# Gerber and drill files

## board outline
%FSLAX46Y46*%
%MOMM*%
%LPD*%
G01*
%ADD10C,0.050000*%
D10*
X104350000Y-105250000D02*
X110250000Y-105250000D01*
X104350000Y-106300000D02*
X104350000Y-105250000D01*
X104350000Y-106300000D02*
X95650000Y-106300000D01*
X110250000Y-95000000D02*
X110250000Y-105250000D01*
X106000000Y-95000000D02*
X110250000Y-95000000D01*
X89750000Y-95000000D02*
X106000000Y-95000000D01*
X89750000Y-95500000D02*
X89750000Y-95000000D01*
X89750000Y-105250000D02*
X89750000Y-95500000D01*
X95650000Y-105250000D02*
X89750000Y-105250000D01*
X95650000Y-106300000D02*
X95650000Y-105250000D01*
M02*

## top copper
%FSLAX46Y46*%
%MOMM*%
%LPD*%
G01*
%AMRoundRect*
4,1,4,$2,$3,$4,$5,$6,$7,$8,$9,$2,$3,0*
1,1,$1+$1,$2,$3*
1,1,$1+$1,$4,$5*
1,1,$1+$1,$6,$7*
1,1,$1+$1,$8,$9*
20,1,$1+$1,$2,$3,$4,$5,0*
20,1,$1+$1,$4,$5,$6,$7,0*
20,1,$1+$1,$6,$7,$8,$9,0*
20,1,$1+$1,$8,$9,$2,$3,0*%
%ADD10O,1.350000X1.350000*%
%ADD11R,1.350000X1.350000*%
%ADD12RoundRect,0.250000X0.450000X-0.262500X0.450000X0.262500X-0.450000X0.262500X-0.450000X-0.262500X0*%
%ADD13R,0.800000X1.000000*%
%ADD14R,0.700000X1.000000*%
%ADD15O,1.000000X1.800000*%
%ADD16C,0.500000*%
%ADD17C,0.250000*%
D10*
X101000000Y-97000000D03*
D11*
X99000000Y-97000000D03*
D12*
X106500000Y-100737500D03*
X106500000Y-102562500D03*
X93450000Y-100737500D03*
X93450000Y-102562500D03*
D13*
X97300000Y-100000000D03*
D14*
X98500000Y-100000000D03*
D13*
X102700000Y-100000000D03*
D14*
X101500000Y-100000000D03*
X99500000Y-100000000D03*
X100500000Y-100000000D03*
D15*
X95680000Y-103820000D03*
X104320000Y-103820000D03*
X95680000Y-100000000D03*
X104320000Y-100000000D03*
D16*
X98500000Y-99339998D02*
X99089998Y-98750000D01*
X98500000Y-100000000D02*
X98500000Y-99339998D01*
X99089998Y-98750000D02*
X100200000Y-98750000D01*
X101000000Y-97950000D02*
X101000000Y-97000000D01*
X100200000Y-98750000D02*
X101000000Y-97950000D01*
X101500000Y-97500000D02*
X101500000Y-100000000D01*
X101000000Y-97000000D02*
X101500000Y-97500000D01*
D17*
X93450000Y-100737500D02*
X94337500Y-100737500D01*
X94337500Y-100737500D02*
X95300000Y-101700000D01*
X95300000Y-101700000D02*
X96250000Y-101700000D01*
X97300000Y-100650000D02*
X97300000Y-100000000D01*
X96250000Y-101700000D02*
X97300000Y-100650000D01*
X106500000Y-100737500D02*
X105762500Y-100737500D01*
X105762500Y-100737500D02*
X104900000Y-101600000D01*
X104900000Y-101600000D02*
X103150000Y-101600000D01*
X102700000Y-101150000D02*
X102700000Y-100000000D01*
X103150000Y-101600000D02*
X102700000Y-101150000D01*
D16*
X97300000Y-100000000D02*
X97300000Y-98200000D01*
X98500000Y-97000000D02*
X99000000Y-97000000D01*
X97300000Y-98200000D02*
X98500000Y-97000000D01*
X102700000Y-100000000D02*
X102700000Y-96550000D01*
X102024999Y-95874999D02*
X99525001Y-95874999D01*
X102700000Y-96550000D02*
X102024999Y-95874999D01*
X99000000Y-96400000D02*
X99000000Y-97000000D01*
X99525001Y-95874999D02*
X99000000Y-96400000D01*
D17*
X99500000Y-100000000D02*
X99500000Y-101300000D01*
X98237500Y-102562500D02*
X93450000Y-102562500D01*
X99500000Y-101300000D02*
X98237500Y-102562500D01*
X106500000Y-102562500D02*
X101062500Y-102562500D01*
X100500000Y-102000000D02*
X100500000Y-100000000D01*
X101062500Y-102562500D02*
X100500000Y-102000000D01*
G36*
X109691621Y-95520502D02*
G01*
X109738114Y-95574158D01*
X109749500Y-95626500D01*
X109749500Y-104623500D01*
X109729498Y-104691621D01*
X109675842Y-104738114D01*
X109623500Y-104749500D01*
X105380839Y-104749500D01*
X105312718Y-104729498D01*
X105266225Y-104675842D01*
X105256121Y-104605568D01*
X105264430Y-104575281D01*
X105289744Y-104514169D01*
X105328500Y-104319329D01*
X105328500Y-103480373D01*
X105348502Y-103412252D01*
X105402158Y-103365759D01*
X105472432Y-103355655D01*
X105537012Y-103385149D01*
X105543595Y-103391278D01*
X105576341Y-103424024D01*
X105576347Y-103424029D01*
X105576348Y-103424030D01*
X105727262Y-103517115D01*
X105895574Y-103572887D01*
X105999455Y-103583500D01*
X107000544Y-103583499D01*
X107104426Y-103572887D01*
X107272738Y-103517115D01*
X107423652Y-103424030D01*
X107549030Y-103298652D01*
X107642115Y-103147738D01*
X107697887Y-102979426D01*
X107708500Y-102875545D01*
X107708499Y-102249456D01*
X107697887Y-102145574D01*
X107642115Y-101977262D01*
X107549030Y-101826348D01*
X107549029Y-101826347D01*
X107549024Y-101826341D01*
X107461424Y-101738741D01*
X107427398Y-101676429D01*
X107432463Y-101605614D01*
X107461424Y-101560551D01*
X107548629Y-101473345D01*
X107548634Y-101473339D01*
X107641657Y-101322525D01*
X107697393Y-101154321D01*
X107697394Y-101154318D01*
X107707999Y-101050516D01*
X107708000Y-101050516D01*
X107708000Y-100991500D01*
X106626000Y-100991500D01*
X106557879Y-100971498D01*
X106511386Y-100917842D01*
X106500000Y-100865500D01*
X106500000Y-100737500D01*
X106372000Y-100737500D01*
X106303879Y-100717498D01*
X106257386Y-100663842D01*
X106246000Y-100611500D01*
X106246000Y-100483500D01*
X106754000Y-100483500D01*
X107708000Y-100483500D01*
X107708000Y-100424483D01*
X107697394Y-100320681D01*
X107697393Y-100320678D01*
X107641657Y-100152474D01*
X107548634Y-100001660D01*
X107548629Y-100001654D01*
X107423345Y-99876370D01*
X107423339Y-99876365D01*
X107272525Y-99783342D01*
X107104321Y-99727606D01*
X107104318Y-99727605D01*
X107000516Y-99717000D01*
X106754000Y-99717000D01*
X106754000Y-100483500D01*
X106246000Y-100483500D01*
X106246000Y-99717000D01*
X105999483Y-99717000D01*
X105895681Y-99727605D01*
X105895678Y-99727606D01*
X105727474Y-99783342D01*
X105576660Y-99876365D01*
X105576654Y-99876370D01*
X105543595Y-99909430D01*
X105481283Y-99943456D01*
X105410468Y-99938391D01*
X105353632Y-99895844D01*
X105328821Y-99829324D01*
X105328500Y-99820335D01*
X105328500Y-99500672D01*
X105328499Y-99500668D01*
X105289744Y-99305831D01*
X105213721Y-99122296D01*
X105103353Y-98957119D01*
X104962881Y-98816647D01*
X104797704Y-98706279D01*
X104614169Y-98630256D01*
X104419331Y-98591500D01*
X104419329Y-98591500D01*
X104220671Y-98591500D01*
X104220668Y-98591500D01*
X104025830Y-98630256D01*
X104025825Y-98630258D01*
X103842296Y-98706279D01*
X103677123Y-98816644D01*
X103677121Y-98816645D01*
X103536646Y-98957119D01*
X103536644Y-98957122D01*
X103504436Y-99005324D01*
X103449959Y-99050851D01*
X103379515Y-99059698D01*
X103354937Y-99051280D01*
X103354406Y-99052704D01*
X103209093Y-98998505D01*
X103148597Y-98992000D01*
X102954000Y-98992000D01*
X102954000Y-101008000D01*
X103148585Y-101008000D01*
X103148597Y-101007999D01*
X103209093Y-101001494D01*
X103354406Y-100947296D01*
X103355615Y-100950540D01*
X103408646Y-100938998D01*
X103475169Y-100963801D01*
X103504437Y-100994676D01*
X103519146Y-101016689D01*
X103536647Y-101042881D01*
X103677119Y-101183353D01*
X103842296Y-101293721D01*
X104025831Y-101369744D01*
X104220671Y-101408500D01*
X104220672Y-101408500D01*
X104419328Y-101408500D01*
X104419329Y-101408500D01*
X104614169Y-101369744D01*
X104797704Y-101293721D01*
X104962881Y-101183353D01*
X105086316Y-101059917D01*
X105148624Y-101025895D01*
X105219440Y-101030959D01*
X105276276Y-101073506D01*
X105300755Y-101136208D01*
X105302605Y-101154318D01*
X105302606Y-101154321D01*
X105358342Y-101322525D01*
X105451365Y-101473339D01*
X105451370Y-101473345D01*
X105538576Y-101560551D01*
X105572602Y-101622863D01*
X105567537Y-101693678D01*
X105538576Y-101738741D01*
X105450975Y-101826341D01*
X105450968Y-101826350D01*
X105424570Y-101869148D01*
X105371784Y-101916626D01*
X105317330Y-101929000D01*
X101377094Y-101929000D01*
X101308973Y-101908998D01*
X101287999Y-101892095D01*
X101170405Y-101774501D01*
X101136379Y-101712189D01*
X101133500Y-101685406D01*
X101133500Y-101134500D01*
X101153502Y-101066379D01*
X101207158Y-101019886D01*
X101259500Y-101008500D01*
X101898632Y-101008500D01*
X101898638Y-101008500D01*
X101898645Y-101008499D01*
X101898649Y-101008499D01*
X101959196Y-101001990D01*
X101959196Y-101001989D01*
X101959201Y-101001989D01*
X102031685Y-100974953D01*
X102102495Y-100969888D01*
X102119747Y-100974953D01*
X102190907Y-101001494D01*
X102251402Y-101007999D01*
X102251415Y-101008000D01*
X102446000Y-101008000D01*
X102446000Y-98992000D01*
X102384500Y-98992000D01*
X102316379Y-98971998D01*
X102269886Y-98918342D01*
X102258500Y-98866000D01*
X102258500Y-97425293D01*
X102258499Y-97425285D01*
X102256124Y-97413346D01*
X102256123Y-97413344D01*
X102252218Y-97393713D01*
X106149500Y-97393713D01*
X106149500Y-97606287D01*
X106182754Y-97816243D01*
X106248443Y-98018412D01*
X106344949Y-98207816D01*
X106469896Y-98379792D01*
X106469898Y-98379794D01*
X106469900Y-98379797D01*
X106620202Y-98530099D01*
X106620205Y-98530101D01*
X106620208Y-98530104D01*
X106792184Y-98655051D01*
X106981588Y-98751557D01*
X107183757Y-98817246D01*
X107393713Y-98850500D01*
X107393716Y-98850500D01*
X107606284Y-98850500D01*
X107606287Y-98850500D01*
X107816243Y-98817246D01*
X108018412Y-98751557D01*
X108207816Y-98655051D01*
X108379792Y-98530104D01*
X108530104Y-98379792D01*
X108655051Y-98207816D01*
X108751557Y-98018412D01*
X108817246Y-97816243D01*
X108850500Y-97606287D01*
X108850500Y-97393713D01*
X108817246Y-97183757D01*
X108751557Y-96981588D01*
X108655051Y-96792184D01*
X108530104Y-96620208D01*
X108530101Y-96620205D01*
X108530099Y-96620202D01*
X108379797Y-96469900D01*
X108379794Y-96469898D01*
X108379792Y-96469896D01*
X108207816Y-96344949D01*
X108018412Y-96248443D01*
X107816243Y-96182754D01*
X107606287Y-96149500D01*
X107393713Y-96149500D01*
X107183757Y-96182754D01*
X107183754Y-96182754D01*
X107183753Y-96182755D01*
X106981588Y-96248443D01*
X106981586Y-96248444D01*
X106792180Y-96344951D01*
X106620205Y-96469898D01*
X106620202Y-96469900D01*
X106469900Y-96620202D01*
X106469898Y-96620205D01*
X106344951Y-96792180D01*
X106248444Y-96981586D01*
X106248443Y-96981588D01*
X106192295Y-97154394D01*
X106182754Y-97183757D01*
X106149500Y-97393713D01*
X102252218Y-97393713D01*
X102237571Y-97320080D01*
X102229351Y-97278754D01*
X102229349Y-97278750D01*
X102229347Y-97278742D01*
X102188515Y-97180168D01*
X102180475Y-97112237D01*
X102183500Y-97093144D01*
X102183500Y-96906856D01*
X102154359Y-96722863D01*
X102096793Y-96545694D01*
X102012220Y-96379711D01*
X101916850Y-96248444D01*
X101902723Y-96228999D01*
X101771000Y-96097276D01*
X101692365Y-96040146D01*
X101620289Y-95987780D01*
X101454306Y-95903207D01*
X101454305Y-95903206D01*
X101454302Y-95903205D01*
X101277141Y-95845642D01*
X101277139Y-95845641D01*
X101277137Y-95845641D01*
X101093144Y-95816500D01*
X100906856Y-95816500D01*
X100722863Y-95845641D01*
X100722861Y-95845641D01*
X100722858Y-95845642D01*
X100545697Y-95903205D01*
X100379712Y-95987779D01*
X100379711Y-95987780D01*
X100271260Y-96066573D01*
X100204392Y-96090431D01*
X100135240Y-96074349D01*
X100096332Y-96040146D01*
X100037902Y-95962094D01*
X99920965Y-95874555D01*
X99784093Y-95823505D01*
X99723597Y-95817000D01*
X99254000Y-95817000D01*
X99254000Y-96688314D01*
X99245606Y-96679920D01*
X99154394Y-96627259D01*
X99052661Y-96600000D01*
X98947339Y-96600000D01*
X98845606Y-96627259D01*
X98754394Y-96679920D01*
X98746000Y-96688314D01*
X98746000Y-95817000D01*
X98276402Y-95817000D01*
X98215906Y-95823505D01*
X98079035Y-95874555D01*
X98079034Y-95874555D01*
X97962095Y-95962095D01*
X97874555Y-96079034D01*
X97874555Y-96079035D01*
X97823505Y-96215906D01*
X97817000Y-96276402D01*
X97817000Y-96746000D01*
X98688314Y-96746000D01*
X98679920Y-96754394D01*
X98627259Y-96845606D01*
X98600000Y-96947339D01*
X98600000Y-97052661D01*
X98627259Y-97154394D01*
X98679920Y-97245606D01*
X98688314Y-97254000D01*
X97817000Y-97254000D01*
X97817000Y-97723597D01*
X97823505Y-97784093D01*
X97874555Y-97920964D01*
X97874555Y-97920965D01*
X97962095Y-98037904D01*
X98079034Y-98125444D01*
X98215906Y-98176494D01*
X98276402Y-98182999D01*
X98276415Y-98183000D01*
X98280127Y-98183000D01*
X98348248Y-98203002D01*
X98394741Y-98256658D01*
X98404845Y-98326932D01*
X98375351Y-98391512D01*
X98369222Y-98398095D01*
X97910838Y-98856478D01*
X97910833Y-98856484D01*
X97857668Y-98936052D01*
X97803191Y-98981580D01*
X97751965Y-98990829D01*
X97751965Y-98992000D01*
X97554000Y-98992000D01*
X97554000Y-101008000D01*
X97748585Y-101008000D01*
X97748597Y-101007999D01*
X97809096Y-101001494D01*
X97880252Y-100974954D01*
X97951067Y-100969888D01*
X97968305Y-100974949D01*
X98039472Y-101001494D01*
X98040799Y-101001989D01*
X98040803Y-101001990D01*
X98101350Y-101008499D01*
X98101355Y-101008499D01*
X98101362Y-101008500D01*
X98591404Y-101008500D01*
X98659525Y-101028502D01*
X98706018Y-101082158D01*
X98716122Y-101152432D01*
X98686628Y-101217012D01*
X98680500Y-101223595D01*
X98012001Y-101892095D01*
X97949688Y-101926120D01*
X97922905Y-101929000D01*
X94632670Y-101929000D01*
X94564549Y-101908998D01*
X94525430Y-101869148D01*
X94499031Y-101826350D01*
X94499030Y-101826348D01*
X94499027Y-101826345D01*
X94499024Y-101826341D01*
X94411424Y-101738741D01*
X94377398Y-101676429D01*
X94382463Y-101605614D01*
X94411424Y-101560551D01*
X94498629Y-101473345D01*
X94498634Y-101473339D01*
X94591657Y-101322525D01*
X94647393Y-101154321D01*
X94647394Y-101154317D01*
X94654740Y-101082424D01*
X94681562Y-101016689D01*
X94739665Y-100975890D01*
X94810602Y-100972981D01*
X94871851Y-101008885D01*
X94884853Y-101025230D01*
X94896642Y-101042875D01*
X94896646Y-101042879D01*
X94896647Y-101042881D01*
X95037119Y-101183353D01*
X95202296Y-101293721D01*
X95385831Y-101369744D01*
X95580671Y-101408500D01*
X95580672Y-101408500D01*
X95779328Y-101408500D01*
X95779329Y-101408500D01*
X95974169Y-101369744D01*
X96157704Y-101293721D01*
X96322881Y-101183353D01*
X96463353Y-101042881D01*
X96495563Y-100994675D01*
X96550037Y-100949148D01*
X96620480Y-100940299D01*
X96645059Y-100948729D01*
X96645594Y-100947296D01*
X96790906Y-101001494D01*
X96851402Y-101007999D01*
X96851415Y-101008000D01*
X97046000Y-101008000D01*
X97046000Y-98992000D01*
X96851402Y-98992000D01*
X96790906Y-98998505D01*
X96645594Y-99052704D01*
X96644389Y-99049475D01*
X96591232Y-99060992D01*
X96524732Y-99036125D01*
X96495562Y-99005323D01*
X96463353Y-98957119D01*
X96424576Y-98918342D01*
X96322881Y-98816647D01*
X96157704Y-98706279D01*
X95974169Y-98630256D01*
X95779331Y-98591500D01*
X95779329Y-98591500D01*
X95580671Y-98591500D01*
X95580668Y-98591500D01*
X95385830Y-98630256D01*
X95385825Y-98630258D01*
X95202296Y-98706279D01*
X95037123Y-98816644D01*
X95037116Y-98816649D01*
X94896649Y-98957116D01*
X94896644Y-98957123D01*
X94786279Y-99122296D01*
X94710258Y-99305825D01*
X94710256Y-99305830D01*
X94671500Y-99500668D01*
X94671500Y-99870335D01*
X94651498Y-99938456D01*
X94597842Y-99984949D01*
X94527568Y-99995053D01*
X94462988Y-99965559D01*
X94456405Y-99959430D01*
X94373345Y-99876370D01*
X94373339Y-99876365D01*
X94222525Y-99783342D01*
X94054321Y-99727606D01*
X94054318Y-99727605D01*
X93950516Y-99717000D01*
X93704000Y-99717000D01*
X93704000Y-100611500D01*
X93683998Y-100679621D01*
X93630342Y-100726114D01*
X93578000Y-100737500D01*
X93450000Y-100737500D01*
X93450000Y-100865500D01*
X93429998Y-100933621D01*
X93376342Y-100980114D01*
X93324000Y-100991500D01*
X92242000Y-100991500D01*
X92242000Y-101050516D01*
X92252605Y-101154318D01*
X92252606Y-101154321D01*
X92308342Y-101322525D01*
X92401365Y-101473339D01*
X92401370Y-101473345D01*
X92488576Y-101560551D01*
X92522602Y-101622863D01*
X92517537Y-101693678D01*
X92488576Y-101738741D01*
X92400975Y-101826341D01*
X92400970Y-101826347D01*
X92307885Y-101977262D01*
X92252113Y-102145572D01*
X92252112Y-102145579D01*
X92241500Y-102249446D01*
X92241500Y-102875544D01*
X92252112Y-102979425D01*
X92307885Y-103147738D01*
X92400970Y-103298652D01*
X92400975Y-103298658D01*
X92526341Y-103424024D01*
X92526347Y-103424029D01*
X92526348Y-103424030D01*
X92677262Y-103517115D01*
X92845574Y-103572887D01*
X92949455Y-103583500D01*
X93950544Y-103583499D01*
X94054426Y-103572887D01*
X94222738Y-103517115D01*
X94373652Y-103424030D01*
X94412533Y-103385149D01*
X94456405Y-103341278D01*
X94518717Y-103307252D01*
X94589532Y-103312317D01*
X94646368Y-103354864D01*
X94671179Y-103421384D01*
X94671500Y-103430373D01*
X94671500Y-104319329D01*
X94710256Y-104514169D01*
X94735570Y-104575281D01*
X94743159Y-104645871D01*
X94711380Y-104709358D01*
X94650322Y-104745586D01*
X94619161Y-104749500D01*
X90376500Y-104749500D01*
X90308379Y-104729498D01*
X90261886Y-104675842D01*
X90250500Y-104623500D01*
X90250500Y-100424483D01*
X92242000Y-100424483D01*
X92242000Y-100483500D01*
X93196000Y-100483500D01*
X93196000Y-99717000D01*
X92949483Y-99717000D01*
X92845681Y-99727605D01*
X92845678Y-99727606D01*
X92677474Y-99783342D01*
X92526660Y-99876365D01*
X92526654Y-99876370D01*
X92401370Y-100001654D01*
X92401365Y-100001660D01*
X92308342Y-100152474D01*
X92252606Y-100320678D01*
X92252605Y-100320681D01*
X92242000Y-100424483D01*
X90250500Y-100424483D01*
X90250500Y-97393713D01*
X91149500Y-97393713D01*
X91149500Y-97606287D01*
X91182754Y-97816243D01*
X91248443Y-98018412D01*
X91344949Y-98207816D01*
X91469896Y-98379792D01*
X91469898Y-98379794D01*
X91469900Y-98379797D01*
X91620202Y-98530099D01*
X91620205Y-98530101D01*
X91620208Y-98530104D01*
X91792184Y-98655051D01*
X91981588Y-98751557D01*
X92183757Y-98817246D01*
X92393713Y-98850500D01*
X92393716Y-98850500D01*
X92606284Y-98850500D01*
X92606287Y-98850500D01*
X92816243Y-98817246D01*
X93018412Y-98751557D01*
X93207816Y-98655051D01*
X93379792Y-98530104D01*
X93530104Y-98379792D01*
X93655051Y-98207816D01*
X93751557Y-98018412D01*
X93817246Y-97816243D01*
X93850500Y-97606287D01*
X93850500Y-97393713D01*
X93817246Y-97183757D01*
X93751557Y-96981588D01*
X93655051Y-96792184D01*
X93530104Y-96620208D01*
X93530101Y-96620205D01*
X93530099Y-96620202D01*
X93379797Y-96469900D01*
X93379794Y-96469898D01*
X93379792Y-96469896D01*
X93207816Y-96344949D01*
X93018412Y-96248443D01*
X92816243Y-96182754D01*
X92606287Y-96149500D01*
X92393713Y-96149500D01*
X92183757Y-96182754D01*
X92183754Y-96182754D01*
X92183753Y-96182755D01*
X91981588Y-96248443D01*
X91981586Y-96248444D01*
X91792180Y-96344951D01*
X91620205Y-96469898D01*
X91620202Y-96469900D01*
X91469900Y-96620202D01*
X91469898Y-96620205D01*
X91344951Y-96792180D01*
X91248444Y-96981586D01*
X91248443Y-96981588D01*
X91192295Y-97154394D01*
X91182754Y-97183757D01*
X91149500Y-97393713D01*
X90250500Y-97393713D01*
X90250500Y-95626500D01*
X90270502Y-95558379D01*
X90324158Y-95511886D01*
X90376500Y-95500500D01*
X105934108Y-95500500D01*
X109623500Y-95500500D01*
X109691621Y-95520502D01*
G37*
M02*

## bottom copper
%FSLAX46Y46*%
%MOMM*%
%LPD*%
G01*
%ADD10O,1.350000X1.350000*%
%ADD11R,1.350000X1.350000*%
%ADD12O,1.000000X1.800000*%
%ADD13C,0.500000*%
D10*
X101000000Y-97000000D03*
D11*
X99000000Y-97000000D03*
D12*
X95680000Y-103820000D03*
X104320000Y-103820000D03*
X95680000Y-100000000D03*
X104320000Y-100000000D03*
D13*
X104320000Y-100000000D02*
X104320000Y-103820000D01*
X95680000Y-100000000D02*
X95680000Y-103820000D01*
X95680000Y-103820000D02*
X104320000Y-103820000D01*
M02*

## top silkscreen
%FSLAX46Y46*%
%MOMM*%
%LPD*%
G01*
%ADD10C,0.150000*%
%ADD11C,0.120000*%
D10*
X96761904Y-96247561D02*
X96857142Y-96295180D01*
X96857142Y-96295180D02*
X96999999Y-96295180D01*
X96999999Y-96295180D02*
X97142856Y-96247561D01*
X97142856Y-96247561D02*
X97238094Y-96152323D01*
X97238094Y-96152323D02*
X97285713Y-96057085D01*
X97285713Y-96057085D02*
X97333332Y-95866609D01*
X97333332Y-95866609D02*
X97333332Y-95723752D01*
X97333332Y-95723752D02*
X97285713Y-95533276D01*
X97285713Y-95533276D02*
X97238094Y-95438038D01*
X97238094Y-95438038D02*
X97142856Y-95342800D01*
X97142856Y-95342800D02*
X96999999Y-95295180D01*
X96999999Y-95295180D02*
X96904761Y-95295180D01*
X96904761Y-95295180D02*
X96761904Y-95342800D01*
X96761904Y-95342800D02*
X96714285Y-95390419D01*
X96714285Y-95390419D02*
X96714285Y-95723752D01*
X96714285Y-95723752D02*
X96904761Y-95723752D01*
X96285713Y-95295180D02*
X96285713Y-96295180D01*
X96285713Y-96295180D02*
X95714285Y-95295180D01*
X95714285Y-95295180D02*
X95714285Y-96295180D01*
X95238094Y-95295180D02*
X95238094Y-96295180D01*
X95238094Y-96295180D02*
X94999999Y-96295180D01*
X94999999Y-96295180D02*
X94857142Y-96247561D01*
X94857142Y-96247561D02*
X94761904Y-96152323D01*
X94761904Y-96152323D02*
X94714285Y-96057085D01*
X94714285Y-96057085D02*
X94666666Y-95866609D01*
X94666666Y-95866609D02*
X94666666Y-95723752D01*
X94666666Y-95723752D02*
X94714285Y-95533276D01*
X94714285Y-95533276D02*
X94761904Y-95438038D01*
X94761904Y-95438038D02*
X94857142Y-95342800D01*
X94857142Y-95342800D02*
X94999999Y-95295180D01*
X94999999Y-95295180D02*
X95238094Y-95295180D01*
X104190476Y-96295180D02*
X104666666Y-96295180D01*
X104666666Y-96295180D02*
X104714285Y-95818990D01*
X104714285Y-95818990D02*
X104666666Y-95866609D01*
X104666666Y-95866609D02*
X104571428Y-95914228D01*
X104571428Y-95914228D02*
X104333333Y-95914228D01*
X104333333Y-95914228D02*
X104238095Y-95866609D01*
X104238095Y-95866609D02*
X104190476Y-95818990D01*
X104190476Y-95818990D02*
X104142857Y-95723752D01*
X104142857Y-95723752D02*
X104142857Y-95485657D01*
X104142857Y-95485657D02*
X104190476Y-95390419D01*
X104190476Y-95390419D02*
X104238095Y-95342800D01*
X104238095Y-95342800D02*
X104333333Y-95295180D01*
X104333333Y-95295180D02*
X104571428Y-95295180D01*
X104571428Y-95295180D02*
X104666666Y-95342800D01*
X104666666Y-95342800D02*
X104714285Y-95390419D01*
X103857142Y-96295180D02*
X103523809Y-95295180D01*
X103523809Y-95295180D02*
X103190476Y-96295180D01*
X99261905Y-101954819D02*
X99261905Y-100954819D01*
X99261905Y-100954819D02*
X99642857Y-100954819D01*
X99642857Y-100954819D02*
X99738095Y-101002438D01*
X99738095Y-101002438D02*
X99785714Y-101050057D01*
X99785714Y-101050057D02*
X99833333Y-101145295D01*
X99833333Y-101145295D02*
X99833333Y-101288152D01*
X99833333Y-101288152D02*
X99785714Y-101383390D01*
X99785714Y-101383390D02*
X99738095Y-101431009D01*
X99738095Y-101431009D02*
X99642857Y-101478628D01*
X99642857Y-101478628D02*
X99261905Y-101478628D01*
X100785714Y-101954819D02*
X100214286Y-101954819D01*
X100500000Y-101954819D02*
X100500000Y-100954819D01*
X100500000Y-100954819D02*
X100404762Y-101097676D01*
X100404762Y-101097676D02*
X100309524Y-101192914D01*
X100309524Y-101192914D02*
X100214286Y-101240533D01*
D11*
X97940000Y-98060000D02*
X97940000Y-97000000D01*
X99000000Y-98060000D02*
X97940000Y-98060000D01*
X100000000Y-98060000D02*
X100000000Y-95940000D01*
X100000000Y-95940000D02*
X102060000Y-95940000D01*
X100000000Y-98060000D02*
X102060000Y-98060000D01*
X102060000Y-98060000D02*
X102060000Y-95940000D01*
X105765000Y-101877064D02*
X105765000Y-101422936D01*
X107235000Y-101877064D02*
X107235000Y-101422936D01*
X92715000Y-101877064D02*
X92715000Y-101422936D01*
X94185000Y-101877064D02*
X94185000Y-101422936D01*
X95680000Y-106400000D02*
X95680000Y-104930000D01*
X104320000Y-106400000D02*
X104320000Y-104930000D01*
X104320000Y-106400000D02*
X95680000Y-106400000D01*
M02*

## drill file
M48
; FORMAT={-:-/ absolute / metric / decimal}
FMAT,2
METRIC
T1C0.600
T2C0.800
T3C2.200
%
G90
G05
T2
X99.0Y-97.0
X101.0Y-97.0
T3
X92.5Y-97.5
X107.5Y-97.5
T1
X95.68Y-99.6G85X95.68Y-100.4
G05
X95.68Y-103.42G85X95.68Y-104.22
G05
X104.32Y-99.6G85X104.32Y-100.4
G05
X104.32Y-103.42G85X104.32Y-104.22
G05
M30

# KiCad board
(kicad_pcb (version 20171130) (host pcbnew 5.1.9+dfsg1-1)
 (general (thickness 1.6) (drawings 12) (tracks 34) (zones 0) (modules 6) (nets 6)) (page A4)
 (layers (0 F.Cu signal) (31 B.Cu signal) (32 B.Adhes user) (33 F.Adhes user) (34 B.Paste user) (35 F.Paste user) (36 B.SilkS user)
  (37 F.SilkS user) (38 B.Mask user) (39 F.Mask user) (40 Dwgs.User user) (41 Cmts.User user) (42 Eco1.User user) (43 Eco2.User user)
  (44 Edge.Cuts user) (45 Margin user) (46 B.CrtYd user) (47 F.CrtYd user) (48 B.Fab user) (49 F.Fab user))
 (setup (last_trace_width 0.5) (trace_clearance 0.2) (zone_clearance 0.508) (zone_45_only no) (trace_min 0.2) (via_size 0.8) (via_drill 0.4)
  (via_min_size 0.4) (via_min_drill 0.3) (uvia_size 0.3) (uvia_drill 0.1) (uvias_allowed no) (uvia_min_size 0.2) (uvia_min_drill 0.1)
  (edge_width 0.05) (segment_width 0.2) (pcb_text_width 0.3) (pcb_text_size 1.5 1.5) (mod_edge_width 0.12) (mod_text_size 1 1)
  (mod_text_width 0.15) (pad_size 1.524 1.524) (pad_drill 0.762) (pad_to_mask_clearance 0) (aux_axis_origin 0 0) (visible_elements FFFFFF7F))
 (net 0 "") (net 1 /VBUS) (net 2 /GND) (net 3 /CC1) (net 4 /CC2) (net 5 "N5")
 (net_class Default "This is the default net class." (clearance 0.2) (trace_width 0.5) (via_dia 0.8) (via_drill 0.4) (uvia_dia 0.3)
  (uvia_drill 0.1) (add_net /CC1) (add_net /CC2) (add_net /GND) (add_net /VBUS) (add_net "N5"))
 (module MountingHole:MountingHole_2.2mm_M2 (layer F.Cu) (at 107.5 97.5)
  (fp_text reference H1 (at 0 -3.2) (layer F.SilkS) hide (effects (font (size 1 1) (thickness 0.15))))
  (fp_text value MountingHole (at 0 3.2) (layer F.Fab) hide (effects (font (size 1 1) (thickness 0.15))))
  (pad 1 np_thru_hole circle (at 0 0) (size 2.2 2.2) (drill 2.2) (layers *.Cu *.Mask)))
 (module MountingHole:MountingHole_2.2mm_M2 (layer F.Cu) (at 92.5 97.5)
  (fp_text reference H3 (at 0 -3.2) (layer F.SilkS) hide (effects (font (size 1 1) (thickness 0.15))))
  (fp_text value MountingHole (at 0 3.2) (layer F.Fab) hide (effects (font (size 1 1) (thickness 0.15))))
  (pad 1 np_thru_hole circle (at 0 0) (size 2.2 2.2) (drill 2.2) (layers *.Cu *.Mask)))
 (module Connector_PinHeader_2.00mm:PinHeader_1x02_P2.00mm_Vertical (layer F.Cu) (at 99 97 90)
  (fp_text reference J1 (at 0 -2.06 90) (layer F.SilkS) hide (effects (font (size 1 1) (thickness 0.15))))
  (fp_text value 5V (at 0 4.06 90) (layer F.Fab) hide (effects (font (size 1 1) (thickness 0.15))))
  (fp_line (start -1.06 -1.06) (end 0 -1.06) (layer F.SilkS) (width 0.12))
  (fp_line (start -1.06 0) (end -1.06 -1.06) (layer F.SilkS) (width 0.12))
  (fp_line (start -1.06 1) (end 1.06 1) (layer F.SilkS) (width 0.12))
  (fp_line (start 1.06 1) (end 1.06 3.06) (layer F.SilkS) (width 0.12))
  (fp_line (start -1.06 1) (end -1.06 3.06) (layer F.SilkS) (width 0.12))
  (fp_line (start -1.06 3.06) (end 1.06 3.06) (layer F.SilkS) (width 0.12))
  (pad 2 thru_hole oval (at 0 2 90) (size 1.35 1.35) (drill 0.8) (layers *.Cu *.Mask) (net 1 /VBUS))
  (pad 1 thru_hole rect (at 0 0 90) (size 1.35 1.35) (drill 0.8) (layers *.Cu *.Mask) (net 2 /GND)))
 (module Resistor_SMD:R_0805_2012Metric (layer F.Cu) (at 106.5 101.65 90)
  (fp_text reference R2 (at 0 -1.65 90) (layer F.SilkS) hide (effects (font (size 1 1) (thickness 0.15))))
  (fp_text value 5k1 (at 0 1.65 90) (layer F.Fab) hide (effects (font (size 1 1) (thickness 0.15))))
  (fp_line (start -0.227064 -0.735) (end 0.227064 -0.735) (layer F.SilkS) (width 0.12))
  (fp_line (start -0.227064 0.735) (end 0.227064 0.735) (layer F.SilkS) (width 0.12))
  (pad 2 smd roundrect (at 0.9125 0 90) (size 1.025 1.4) (layers F.Cu F.Paste F.Mask) (roundrect_rratio 0.243902) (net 2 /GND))
  (pad 1 smd roundrect (at -0.9125 0 90) (size 1.025 1.4) (layers F.Cu F.Paste F.Mask) (roundrect_rratio 0.243902) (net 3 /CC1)))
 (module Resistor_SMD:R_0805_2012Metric (layer F.Cu) (at 93.45 101.65 90)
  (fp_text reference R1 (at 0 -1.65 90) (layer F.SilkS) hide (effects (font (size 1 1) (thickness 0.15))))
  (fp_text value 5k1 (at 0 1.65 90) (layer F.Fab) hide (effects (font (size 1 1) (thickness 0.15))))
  (fp_line (start -0.227064 -0.735) (end 0.227064 -0.735) (layer F.SilkS) (width 0.12))
  (fp_line (start -0.227064 0.735) (end 0.227064 0.735) (layer F.SilkS) (width 0.12))
  (pad 2 smd roundrect (at 0.9125 0 90) (size 1.025 1.4) (layers F.Cu F.Paste F.Mask) (roundrect_rratio 0.243902) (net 2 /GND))
  (pad 1 smd roundrect (at -0.9125 0 90) (size 1.025 1.4) (layers F.Cu F.Paste F.Mask) (roundrect_rratio 0.243902) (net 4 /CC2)))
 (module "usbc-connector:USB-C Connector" (layer F.Cu) (at 100 100)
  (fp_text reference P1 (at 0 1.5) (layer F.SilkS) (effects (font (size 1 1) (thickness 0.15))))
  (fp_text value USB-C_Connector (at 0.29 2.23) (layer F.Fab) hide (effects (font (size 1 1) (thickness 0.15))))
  (fp_line (start -4.32 6.4) (end -4.32 4.93) (layer F.SilkS) (width 0.12))
  (fp_line (start 4.32 6.4) (end 4.32 4.93) (layer F.SilkS) (width 0.12))
  (fp_line (start 4.32 6.4) (end -4.32 6.4) (layer F.SilkS) (width 0.12))
  (pad B12 smd rect (at -2.7 0) (size 0.8 1) (layers F.Cu F.Paste F.Mask) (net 2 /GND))
  (pad B9 smd rect (at -1.5 0) (size 0.7 1) (layers F.Cu F.Paste F.Mask) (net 1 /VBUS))
  (pad A12 smd rect (at 2.7 0) (size 0.8 1) (layers F.Cu F.Paste F.Mask) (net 2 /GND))
  (pad A9 smd rect (at 1.5 0) (size 0.7 1) (layers F.Cu F.Paste F.Mask) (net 1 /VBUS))
  (pad B5 smd rect (at -0.5 0) (size 0.7 1) (layers F.Cu F.Paste F.Mask) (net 4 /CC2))
  (pad A5 smd rect (at 0.5 0) (size 0.7 1) (layers F.Cu F.Paste F.Mask) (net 3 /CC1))
  (pad 5 thru_hole oval (at -4.32 3.82) (size 1 1.8) (drill oval 0.6 1.4) (layers *.Cu *.Mask) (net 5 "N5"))
  (pad 5 thru_hole oval (at 4.32 3.82) (size 1 1.8) (drill oval 0.6 1.4) (layers *.Cu *.Mask) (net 5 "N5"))
  (pad 5 thru_hole oval (at -4.32 0) (size 1 1.8) (drill oval 0.6 1.4) (layers *.Cu *.Mask) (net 5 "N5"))
  (pad 5 thru_hole oval (at 4.32 0) (size 1 1.8) (drill oval 0.6 1.4) (layers *.Cu *.Mask) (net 5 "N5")))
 (gr_line (start 104.35 105.25) (end 110.25 105.25) (layer Edge.Cuts) (width 0.05))
 (gr_line (start 104.35 106.3) (end 104.35 105.25) (layer Edge.Cuts) (width 0.05))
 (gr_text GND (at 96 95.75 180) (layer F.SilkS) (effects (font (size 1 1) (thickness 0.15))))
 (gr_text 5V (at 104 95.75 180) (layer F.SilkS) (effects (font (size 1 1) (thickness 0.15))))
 (gr_line (start 104.35 106.3) (end 95.65 106.3) (layer Edge.Cuts) (width 0.05))
 (gr_line (start 110.25 95) (end 110.25 105.25) (layer Edge.Cuts) (width 0.05))
 (gr_line (start 106 95) (end 110.25 95) (layer Edge.Cuts) (width 0.05))
 (gr_line (start 89.75 95) (end 106 95) (layer Edge.Cuts) (width 0.05))
 (gr_line (start 89.75 95.5) (end 89.75 95) (layer Edge.Cuts) (width 0.05))
 (gr_line (start 89.75 105.25) (end 89.75 95.5) (layer Edge.Cuts) (width 0.05))
 (gr_line (start 95.65 105.25) (end 89.75 105.25) (layer Edge.Cuts) (width 0.05))
 (gr_line (start 95.65 106.3) (end 95.65 105.25) (layer Edge.Cuts) (width 0.05))
 (segment (start 98.5 99.339998) (end 99.089998 98.75) (width 0.5) (layer F.Cu) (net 1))
 (segment (start 98.5 100) (end 98.5 99.339998) (width 0.5) (layer F.Cu) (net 1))
 (segment (start 99.089998 98.75) (end 100.2 98.75) (width 0.5) (layer F.Cu) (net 1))
 (segment (start 101 97.95) (end 101 97) (width 0.5) (layer F.Cu) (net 1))
 (segment (start 100.2 98.75) (end 101 97.95) (width 0.5) (layer F.Cu) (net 1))
 (segment (start 101.5 97.5) (end 101.5 100) (width 0.5) (layer F.Cu) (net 1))
 (segment (start 101 97) (end 101.5 97.5) (width 0.5) (layer F.Cu) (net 1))
 (segment (start 93.45 100.7375) (end 94.3375 100.7375) (width 0.25) (layer F.Cu) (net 2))
 (segment (start 94.3375 100.7375) (end 95.3 101.7) (width 0.25) (layer F.Cu) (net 2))
 (segment (start 95.3 101.7) (end 96.25 101.7) (width 0.25) (layer F.Cu) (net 2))
 (segment (start 97.3 100.65) (end 97.3 100) (width 0.25) (layer F.Cu) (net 2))
 (segment (start 96.25 101.7) (end 97.3 100.65) (width 0.25) (layer F.Cu) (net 2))
 (segment (start 106.5 100.7375) (end 105.7625 100.7375) (width 0.25) (layer F.Cu) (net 2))
 (segment (start 105.7625 100.7375) (end 104.9 101.6) (width 0.25) (layer F.Cu) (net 2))
 (segment (start 104.9 101.6) (end 103.15 101.6) (width 0.25) (layer F.Cu) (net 2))
 (segment (start 102.7 101.15) (end 102.7 100) (width 0.25) (layer F.Cu) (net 2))
 (segment (start 103.15 101.6) (end 102.7 101.15) (width 0.25) (layer F.Cu) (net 2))
 (segment (start 97.3 100) (end 97.3 98.2) (width 0.5) (layer F.Cu) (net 2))
 (segment (start 98.5 97) (end 99 97) (width 0.5) (layer F.Cu) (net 2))
 (segment (start 97.3 98.2) (end 98.5 97) (width 0.5) (layer F.Cu) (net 2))
 (segment (start 102.7 100) (end 102.7 96.55) (width 0.5) (layer F.Cu) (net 2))
 (segment (start 102.024999 95.874999) (end 99.525001 95.874999) (width 0.5) (layer F.Cu) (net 2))
 (segment (start 102.7 96.55) (end 102.024999 95.874999) (width 0.5) (layer F.Cu) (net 2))
 (segment (start 99 96.4) (end 99 97) (width 0.5) (layer F.Cu) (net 2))
 (segment (start 99.525001 95.874999) (end 99 96.4) (width 0.5) (layer F.Cu) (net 2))
 (segment (start 99.5 100) (end 99.5 101.3) (width 0.25) (layer F.Cu) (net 4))
 (segment (start 98.2375 102.5625) (end 93.45 102.5625) (width 0.25) (layer F.Cu) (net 4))
 (segment (start 99.5 101.3) (end 98.2375 102.5625) (width 0.25) (layer F.Cu) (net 4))
 (segment (start 106.5 102.5625) (end 101.0625 102.5625) (width 0.25) (layer F.Cu) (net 3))
 (segment (start 100.5 102) (end 100.5 100) (width 0.25) (layer F.Cu) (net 3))
 (segment (start 101.0625 102.5625) (end 100.5 102) (width 0.25) (layer F.Cu) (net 3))
 (segment (start 104.32 100) (end 104.32 103.82) (width 0.5) (layer B.Cu) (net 5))
 (segment (start 95.68 100) (end 95.68 103.82) (width 0.5) (layer B.Cu) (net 5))
 (segment (start 95.68 103.82) (end 104.32 103.82) (width 0.5) (layer B.Cu) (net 5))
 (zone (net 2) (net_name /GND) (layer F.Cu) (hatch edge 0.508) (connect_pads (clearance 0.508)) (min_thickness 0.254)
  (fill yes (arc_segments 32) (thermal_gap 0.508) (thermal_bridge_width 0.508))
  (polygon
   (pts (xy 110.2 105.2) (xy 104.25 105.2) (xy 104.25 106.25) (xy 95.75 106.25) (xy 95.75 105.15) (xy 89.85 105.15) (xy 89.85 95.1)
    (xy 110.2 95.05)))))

